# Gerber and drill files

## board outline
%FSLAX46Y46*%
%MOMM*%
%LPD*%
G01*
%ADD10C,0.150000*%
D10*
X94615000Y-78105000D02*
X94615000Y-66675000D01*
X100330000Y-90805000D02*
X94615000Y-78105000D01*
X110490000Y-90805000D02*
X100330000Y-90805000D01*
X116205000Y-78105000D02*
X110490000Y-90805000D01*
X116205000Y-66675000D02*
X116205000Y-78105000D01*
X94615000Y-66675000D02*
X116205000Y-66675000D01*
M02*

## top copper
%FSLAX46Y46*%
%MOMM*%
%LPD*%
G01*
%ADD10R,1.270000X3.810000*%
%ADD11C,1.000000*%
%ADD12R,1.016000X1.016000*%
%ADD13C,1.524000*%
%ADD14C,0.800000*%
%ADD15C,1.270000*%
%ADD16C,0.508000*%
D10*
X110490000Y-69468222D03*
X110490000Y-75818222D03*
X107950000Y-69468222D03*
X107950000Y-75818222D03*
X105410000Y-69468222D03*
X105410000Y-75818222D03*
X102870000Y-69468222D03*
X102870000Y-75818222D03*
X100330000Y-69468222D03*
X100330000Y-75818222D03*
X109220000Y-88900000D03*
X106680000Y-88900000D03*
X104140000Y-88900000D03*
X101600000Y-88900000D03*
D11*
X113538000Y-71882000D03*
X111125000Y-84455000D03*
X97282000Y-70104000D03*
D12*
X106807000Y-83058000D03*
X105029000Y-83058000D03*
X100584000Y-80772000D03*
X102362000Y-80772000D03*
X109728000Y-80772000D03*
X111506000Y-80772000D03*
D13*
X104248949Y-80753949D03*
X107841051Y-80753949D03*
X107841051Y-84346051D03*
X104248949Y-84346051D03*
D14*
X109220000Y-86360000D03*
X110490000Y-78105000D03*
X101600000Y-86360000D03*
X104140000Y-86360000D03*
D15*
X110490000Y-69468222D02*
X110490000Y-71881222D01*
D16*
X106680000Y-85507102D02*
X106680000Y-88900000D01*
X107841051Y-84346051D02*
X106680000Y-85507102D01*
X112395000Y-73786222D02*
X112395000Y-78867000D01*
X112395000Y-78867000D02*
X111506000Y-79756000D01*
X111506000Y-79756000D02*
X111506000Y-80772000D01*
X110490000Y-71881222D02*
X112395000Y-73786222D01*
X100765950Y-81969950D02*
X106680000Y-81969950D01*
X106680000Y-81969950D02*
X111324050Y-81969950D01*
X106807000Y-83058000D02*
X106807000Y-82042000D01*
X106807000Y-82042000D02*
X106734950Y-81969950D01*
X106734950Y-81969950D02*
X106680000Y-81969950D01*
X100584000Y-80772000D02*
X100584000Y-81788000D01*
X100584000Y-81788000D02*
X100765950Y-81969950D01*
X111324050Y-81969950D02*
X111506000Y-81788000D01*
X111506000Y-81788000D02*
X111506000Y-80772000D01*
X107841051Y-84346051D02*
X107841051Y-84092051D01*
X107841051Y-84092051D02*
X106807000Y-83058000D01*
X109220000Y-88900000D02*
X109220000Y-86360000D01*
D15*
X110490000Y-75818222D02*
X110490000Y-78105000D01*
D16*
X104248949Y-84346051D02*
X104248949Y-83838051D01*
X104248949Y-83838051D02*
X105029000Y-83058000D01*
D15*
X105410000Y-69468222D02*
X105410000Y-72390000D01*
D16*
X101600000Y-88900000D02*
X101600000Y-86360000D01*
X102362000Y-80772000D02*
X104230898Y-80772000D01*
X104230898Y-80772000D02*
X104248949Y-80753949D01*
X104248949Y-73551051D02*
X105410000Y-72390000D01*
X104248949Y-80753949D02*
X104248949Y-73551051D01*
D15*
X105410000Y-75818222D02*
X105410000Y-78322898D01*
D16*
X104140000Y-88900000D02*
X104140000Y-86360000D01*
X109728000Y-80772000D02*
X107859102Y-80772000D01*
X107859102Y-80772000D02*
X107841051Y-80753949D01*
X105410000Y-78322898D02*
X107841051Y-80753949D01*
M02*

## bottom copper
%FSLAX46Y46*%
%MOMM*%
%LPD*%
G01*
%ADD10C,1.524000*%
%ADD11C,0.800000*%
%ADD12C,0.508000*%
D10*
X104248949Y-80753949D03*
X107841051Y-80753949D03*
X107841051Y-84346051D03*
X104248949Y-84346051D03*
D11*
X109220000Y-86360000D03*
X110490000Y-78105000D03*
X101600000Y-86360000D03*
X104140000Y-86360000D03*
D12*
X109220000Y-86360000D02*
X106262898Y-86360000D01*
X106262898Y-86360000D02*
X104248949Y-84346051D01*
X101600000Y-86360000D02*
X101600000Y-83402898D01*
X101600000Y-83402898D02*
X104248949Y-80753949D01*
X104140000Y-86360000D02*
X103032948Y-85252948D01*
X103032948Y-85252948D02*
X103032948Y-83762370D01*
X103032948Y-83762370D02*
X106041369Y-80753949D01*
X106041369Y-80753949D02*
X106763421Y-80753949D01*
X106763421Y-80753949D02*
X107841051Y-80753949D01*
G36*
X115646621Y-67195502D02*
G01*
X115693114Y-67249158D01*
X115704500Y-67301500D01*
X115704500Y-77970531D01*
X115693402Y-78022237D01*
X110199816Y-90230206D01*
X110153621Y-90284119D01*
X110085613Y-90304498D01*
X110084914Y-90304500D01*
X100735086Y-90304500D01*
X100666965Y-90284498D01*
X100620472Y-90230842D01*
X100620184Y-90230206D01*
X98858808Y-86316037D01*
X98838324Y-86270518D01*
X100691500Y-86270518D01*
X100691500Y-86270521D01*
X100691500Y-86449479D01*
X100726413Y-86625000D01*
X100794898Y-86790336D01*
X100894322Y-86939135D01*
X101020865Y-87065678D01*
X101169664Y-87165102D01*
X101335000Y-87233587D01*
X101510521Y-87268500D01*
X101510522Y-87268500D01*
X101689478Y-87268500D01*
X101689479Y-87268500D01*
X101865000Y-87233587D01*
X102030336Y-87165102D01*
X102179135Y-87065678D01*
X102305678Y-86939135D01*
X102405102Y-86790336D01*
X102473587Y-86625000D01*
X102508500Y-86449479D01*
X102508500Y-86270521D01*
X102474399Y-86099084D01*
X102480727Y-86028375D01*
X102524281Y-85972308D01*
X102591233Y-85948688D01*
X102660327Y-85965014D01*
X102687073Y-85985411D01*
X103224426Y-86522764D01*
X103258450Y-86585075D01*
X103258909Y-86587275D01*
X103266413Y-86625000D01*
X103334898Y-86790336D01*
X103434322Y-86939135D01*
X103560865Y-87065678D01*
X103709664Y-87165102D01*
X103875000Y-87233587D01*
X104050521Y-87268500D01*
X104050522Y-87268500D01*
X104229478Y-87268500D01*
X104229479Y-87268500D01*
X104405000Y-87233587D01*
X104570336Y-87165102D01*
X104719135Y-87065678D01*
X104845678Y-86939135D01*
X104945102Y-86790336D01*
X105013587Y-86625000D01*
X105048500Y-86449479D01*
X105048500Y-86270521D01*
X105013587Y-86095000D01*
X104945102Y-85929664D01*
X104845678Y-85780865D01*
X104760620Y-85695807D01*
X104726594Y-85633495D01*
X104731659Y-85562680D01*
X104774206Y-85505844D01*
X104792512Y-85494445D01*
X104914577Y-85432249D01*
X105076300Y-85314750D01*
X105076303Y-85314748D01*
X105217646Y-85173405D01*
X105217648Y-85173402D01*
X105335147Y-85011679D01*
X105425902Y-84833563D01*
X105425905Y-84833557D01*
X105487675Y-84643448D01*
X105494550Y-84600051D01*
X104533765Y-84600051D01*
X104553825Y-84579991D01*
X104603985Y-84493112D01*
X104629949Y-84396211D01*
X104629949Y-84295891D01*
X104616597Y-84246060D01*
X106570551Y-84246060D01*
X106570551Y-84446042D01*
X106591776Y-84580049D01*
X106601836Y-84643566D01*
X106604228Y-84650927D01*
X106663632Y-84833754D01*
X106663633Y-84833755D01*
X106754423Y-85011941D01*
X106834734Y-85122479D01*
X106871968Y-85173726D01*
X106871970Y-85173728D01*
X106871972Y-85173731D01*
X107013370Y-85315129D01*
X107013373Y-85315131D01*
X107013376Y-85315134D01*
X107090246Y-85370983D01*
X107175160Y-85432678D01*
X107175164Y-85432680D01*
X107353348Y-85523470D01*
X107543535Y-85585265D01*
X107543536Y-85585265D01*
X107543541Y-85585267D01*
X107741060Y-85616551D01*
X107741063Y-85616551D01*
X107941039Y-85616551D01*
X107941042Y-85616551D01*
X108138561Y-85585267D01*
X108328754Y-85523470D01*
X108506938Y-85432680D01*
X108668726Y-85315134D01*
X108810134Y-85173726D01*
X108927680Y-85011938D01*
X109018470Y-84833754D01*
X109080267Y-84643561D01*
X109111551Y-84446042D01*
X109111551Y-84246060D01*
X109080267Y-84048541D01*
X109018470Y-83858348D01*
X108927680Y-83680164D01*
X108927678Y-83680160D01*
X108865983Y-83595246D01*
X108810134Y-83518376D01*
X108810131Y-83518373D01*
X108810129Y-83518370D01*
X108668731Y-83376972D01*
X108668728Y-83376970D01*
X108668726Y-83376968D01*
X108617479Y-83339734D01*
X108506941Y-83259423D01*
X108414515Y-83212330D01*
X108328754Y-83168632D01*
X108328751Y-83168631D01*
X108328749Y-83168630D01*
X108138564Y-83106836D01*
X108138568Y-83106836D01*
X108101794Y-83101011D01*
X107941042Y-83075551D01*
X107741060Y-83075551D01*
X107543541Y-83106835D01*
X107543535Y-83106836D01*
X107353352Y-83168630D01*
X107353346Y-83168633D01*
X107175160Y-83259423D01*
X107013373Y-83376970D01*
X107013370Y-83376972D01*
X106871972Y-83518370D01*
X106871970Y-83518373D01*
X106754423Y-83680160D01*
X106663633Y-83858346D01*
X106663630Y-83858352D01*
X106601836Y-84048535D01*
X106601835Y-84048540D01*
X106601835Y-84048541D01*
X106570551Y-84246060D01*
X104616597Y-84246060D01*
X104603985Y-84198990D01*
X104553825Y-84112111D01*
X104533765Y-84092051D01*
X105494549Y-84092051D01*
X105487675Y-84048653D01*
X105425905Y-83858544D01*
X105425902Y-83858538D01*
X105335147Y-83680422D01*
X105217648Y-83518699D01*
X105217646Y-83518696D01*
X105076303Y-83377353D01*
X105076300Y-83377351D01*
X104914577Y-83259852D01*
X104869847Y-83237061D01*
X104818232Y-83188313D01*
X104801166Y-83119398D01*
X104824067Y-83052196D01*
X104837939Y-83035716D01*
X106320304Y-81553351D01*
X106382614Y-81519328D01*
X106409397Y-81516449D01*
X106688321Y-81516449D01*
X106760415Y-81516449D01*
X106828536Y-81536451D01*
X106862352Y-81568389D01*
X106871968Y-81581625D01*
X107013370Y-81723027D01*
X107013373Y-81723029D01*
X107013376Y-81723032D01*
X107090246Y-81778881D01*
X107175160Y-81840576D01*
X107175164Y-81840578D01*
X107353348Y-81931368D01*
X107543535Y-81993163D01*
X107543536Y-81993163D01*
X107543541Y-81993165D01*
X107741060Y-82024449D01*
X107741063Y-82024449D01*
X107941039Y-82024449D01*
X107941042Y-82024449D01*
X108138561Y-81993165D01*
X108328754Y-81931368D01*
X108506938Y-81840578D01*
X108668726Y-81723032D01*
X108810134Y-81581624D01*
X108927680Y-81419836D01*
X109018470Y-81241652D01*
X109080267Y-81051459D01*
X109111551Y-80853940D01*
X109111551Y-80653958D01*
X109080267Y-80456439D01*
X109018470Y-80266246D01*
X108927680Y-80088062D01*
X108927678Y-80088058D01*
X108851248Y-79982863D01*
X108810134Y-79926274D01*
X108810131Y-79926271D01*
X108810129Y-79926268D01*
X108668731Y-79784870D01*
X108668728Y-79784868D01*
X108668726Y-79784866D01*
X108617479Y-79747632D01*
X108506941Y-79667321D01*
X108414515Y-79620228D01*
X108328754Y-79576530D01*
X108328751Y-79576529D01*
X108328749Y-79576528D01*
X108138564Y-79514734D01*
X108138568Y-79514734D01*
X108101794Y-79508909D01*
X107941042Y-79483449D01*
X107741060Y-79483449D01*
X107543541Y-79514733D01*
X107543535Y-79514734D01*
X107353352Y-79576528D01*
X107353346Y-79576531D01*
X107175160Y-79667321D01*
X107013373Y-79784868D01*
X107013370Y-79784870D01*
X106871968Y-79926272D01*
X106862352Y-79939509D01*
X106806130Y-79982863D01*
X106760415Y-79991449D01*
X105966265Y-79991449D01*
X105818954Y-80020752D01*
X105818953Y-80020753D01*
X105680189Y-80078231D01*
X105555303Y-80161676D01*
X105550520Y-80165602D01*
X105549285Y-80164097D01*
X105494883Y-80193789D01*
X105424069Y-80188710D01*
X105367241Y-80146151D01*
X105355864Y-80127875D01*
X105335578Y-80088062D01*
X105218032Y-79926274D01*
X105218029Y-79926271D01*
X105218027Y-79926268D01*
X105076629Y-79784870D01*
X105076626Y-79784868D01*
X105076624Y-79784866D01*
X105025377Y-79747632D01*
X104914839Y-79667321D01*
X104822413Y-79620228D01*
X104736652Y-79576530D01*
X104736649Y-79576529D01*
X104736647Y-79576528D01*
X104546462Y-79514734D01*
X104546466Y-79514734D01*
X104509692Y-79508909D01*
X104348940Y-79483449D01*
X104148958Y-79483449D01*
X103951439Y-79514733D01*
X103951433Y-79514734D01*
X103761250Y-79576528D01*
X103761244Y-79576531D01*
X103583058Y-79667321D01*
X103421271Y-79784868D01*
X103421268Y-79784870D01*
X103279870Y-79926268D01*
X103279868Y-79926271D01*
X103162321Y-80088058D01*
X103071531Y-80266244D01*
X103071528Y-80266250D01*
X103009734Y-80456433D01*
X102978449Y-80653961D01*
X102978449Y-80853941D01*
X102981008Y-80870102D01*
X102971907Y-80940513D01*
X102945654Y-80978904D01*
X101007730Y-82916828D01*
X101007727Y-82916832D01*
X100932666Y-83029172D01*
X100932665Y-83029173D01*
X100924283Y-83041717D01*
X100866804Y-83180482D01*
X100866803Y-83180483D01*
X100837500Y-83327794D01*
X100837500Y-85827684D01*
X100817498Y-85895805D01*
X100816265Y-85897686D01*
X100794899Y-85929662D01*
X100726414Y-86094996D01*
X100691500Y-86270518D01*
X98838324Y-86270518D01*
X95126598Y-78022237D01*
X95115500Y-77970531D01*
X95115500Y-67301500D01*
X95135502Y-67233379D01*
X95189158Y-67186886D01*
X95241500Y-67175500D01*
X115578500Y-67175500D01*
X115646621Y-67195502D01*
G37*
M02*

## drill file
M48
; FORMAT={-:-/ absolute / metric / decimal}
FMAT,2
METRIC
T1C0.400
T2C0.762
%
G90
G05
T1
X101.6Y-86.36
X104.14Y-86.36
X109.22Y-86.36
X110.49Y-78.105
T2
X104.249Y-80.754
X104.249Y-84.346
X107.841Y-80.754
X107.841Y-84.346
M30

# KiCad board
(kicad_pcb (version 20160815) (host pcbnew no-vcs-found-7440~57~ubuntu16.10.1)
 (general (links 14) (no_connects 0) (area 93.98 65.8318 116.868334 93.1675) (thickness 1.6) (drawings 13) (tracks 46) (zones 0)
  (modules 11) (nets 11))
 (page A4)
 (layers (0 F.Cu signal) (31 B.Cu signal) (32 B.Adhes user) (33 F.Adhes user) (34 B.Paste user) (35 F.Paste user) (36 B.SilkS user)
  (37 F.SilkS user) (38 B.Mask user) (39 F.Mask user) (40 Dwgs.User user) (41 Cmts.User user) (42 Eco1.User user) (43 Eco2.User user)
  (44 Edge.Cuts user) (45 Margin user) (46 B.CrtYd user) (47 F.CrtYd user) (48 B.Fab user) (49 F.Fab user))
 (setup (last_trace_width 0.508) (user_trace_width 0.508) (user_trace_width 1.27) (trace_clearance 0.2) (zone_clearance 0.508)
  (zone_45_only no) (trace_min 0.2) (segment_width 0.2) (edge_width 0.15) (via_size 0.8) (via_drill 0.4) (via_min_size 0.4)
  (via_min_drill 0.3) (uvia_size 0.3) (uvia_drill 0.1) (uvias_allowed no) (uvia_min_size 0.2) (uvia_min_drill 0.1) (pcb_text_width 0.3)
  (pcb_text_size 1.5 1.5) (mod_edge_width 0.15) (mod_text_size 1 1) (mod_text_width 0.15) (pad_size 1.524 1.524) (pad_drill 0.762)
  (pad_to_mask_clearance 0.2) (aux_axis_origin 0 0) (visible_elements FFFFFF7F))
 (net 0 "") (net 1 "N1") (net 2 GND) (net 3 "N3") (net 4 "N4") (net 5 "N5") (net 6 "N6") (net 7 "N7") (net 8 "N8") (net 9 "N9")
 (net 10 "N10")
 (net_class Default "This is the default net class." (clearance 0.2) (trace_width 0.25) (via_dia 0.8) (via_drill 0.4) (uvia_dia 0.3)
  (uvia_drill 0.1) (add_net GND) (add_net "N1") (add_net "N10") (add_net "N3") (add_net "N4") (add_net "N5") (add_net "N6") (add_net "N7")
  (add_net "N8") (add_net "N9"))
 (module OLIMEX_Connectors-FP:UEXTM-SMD (layer F.Cu) (at 105.41 72.643222)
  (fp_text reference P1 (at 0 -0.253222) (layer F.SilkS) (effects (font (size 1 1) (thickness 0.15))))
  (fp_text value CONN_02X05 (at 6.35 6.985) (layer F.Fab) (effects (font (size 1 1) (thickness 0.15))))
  (pad 1 smd rect (at 5.08 -3.175) (size 1.27 3.81) (layers F.Cu F.Paste F.Mask) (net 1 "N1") (solder_mask_margin 0.0508)
   (solder_paste_margin -0.0508) (clearance 0.0508))
  (pad 2 smd rect (at 5.08 3.175) (size 1.27 3.81) (layers F.Cu F.Paste F.Mask) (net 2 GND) (solder_mask_margin 0.0508)
   (solder_paste_margin -0.0508) (clearance 0.0508))
  (pad 3 smd rect (at 2.54 -3.175) (size 1.27 3.81) (layers F.Cu F.Paste F.Mask) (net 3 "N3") (solder_mask_margin 0.0508)
   (solder_paste_margin -0.0508) (clearance 0.0508))
  (pad 4 smd rect (at 2.54 3.175) (size 1.27 3.81) (layers F.Cu F.Paste F.Mask) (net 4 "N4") (solder_mask_margin 0.0508)
   (solder_paste_margin -0.0508) (clearance 0.0508))
  (pad 5 smd rect (at 0 -3.175) (size 1.27 3.81) (layers F.Cu F.Paste F.Mask) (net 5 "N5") (solder_mask_margin 0.0508)
   (solder_paste_margin -0.0508) (clearance 0.0508))
  (pad 6 smd rect (at 0 3.175) (size 1.27 3.81) (layers F.Cu F.Paste F.Mask) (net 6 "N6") (solder_mask_margin 0.0508)
   (solder_paste_margin -0.0508) (clearance 0.0508))
  (pad 7 smd rect (at -2.54 -3.175) (size 1.27 3.81) (layers F.Cu F.Paste F.Mask) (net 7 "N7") (solder_mask_margin 0.0508)
   (solder_paste_margin -0.0508) (clearance 0.0508))
  (pad 8 smd rect (at -2.54 3.175) (size 1.27 3.81) (layers F.Cu F.Paste F.Mask) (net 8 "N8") (solder_mask_margin 0.0508)
   (solder_paste_margin -0.0508) (clearance 0.0508))
  (pad 9 smd rect (at -5.08 -3.175) (size 1.27 3.81) (layers F.Cu F.Paste F.Mask) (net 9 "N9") (solder_mask_margin 0.0508)
   (solder_paste_margin -0.0508) (clearance 0.0508))
  (pad 10 smd rect (at -5.08 3.175) (size 1.27 3.81) (layers F.Cu F.Paste F.Mask) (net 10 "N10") (solder_mask_margin 0.0508)
   (solder_paste_margin -0.0508) (clearance 0.0508)))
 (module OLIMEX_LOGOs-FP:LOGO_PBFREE (layer F.Cu) (at 98.044 80.01)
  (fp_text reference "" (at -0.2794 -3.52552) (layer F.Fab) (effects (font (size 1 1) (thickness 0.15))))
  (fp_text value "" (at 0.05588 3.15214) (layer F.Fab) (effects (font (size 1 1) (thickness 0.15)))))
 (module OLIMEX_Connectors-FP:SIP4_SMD (layer F.Cu) (at 105.41 88.9 180)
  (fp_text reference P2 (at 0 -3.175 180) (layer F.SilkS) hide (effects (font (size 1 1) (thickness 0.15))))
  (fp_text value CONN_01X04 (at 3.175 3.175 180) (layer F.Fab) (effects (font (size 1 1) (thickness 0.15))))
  (pad 1 smd rect (at -3.81 0 180) (size 1.27 3.81) (layers F.Cu F.Mask) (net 2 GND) (solder_mask_margin 0.0508)
   (solder_paste_margin -0.0508) (clearance 0.0508))
  (pad 2 smd rect (at -1.27 0 180) (size 1.27 3.81) (layers F.Cu F.Mask) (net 1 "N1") (solder_mask_margin 0.0508)
   (solder_paste_margin -0.0508) (clearance 0.0508))
  (pad 3 smd rect (at 1.27 0 180) (size 1.27 3.81) (layers F.Cu F.Mask) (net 6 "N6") (solder_mask_margin 0.0508)
   (solder_paste_margin -0.0508) (clearance 0.0508))
  (pad 4 smd rect (at 3.81 0 180) (size 1.27 3.81) (layers F.Cu F.Mask) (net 5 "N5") (solder_mask_margin 0.0508)
   (solder_paste_margin -0.0508) (clearance 0.0508)))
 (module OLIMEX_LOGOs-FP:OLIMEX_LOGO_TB (layer B.Cu) (at 105.41 69.85 180)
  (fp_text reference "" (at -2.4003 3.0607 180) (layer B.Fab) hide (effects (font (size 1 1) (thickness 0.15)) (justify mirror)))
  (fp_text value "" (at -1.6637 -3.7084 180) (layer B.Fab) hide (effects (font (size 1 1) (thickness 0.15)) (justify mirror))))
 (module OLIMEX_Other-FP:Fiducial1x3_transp (layer F.Cu) (at 113.538 71.882)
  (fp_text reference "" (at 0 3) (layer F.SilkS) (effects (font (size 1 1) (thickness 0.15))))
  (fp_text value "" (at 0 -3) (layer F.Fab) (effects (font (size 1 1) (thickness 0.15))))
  (pad Fid1 connect circle (at 0 0) (size 1 1) (layers F.Cu F.Mask) (solder_mask_margin 0.127) (clearance 1.016) (zone_connect 0)))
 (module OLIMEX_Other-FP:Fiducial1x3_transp (layer F.Cu) (at 111.125 84.455)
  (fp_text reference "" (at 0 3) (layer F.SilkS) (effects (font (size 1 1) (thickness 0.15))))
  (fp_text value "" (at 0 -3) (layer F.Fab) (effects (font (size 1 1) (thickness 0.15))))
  (pad Fid1 connect circle (at 0 0) (size 1 1) (layers F.Cu F.Mask) (solder_mask_margin 0.127) (clearance 1.016) (zone_connect 0)))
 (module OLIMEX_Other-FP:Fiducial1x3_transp (layer F.Cu) (at 97.282 70.104)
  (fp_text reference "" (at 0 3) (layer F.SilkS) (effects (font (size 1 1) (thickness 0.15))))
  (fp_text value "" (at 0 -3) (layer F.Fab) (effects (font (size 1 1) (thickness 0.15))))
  (pad Fid1 connect circle (at 0 0) (size 1 1) (layers F.Cu F.Mask) (solder_mask_margin 0.127) (clearance 1.016) (zone_connect 0)))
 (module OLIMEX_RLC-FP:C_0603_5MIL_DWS (layer F.Cu) (at 105.918 83.058 180)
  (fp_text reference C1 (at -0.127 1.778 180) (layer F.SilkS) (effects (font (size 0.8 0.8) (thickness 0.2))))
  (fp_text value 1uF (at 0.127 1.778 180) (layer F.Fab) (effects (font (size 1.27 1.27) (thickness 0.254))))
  (pad 1 smd rect (at -0.889 0 180) (size 1.016 1.016) (layers F.Cu F.Paste F.Mask) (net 1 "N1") (solder_mask_margin 0.0508)
   (clearance 0.0508))
  (pad 2 smd rect (at 0.889 0 180) (size 1.016 1.016) (layers F.Cu F.Paste F.Mask) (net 2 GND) (solder_mask_margin 0.0508)
   (clearance 0.0508)))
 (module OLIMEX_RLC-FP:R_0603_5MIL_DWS (layer F.Cu) (at 101.473 80.772)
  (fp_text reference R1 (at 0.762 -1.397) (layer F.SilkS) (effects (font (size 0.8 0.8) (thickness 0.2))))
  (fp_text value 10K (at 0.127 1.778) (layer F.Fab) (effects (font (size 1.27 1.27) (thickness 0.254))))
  (pad 1 smd rect (at -0.889 0) (size 1.016 1.016) (layers F.Cu F.Paste F.Mask) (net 1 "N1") (solder_mask_margin 0.0508))
  (pad 2 smd rect (at 0.889 0) (size 1.016 1.016) (layers F.Cu F.Paste F.Mask) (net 5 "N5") (solder_mask_margin 0.0508)))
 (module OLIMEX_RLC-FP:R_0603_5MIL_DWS (layer F.Cu) (at 110.617 80.772 180)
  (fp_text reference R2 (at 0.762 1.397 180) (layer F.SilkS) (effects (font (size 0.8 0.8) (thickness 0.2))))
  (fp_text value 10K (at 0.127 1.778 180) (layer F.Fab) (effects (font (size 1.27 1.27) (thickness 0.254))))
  (pad 2 smd rect (at 0.889 0 180) (size 1.016 1.016) (layers F.Cu F.Paste F.Mask) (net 6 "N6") (solder_mask_margin 0.0508))
  (pad 1 smd rect (at -0.889 0 180) (size 1.016 1.016) (layers F.Cu F.Paste F.Mask) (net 1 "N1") (solder_mask_margin 0.0508)))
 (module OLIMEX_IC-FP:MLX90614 (layer B.Cu) (at 106.045 82.55 225)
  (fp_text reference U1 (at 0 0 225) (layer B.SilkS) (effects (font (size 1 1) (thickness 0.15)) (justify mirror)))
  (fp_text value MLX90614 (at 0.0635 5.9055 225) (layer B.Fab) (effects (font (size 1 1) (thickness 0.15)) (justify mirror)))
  (pad 1 thru_hole circle (at 0 2.54 225) (size 1.524 1.524) (drill 0.762) (layers *.Cu *.Mask) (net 5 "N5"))
  (pad 2 thru_hole circle (at -2.54 0 225) (size 1.524 1.524) (drill 0.762) (layers *.Cu *.Mask) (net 6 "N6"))
  (pad 3 thru_hole circle (at 0 -2.54 225) (size 1.524 1.524) (drill 0.762) (layers *.Cu *.Mask) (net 1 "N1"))
  (pad 4 thru_hole circle (at 2.54 0 225) (size 1.524 1.524) (drill 0.762) (layers *.Cu *.Mask) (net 2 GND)))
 (gr_line (start 94.615 78.105) (end 94.615 66.675) (layer Edge.Cuts) (width 0.15))
 (gr_line (start 100.33 90.805) (end 94.615 78.105) (layer Edge.Cuts) (width 0.15))
 (gr_line (start 110.49 90.805) (end 100.33 90.805) (layer Edge.Cuts) (width 0.15))
 (gr_line (start 116.205 78.105) (end 110.49 90.805) (layer Edge.Cuts) (width 0.15))
 (gr_line (start 116.205 66.675) (end 116.205 78.105) (layer Edge.Cuts) (width 0.15))
 (gr_line (start 94.615 66.675) (end 116.205 66.675) (layer Edge.Cuts) (width 0.15))
 (segment (start 110.49 69.468222) (end 110.49 71.881222) (width 1.27) (layer F.Cu) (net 1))
 (segment (start 106.68 85.507102) (end 106.68 88.9) (width 0.508) (layer F.Cu) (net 1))
 (segment (start 107.841051 84.346051) (end 106.68 85.507102) (width 0.508) (layer F.Cu) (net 1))
 (segment (start 112.395 73.786222) (end 112.395 78.867) (width 0.508) (layer F.Cu) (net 1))
 (segment (start 112.395 78.867) (end 111.506 79.756) (width 0.508) (layer F.Cu) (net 1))
 (segment (start 111.506 79.756) (end 111.506 80.772) (width 0.508) (layer F.Cu) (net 1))
 (segment (start 110.49 71.881222) (end 112.395 73.786222) (width 0.508) (layer F.Cu) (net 1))
 (segment (start 100.76595 81.96995) (end 106.68 81.96995) (width 0.508) (layer F.Cu) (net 1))
 (segment (start 106.68 81.96995) (end 111.32405 81.96995) (width 0.508) (layer F.Cu) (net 1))
 (segment (start 106.807 83.058) (end 106.807 82.042) (width 0.508) (layer F.Cu) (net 1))
 (segment (start 106.807 82.042) (end 106.73495 81.96995) (width 0.508) (layer F.Cu) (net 1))
 (segment (start 106.73495 81.96995) (end 106.68 81.96995) (width 0.508) (layer F.Cu) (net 1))
 (segment (start 100.584 80.772) (end 100.584 81.788) (width 0.508) (layer F.Cu) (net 1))
 (segment (start 100.584 81.788) (end 100.76595 81.96995) (width 0.508) (layer F.Cu) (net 1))
 (segment (start 111.32405 81.96995) (end 111.506 81.788) (width 0.508) (layer F.Cu) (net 1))
 (segment (start 111.506 81.788) (end 111.506 80.772) (width 0.508) (layer F.Cu) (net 1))
 (segment (start 107.841051 84.346051) (end 107.841051 84.092051) (width 0.508) (layer F.Cu) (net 1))
 (segment (start 107.841051 84.092051) (end 106.807 83.058) (width 0.508) (layer F.Cu) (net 1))
 (segment (start 109.22 86.36) (end 106.262898 86.36) (width 0.508) (layer B.Cu) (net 2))
 (segment (start 106.262898 86.36) (end 104.248949 84.346051) (width 0.508) (layer B.Cu) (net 2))
 (segment (start 109.22 88.9) (end 109.22 86.36) (width 0.508) (layer F.Cu) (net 2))
 (via (at 109.22 86.36) (size 0.8) (drill 0.4) (layers F.Cu B.Cu) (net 2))
 (segment (start 110.49 75.818222) (end 110.49 78.105) (width 1.27) (layer F.Cu) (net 2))
 (via (at 110.49 78.105) (size 0.8) (drill 0.4) (layers F.Cu B.Cu) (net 2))
 (segment (start 104.248949 84.346051) (end 104.248949 83.838051) (width 0.508) (layer F.Cu) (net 2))
 (segment (start 104.248949 83.838051) (end 105.029 83.058) (width 0.508) (layer F.Cu) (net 2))
 (segment (start 105.41 69.468222) (end 105.41 72.39) (width 1.27) (layer F.Cu) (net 5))
 (segment (start 101.6 86.36) (end 101.6 83.402898) (width 0.508) (layer B.Cu) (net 5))
 (segment (start 101.6 83.402898) (end 104.248949 80.753949) (width 0.508) (layer B.Cu) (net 5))
 (segment (start 101.6 88.9) (end 101.6 86.36) (width 0.508) (layer F.Cu) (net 5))
 (via (at 101.6 86.36) (size 0.8) (drill 0.4) (layers F.Cu B.Cu) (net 5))
 (segment (start 102.362 80.772) (end 104.230898 80.772) (width 0.508) (layer F.Cu) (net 5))
 (segment (start 104.230898 80.772) (end 104.248949 80.753949) (width 0.508) (layer F.Cu) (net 5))
 (segment (start 104.248949 73.551051) (end 105.41 72.39) (width 0.508) (layer F.Cu) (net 5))
 (segment (start 104.248949 80.753949) (end 104.248949 73.551051) (width 0.508) (layer F.Cu) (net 5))
 (segment (start 105.41 75.818222) (end 105.41 78.322898) (width 1.27) (layer F.Cu) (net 6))
 (segment (start 104.14 86.36) (end 103.032948 85.252948) (width 0.508) (layer B.Cu) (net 6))
 (segment (start 103.032948 85.252948) (end 103.032948 83.76237) (width 0.508) (layer B.Cu) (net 6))
 (segment (start 103.032948 83.76237) (end 106.041369 80.753949) (width 0.508) (layer B.Cu) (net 6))
 (segment (start 106.041369 80.753949) (end 106.763421 80.753949) (width 0.508) (layer B.Cu) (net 6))
 (segment (start 106.763421 80.753949) (end 107.841051 80.753949) (width 0.508) (layer B.Cu) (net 6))
 (segment (start 104.14 88.9) (end 104.14 86.36) (width 0.508) (layer F.Cu) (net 6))
 (via (at 104.14 86.36) (size 0.8) (drill 0.4) (layers F.Cu B.Cu) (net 6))
 (segment (start 109.728 80.772) (end 107.859102 80.772) (width 0.508) (layer F.Cu) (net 6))
 (segment (start 107.859102 80.772) (end 107.841051 80.753949) (width 0.508) (layer F.Cu) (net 6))
 (segment (start 105.41 78.322898) (end 107.841051 80.753949) (width 0.508) (layer F.Cu) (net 6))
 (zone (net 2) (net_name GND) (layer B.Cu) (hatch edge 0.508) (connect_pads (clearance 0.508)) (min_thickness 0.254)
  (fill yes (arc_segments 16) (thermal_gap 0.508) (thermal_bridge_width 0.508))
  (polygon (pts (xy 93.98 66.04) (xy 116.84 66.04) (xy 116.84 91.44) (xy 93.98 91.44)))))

